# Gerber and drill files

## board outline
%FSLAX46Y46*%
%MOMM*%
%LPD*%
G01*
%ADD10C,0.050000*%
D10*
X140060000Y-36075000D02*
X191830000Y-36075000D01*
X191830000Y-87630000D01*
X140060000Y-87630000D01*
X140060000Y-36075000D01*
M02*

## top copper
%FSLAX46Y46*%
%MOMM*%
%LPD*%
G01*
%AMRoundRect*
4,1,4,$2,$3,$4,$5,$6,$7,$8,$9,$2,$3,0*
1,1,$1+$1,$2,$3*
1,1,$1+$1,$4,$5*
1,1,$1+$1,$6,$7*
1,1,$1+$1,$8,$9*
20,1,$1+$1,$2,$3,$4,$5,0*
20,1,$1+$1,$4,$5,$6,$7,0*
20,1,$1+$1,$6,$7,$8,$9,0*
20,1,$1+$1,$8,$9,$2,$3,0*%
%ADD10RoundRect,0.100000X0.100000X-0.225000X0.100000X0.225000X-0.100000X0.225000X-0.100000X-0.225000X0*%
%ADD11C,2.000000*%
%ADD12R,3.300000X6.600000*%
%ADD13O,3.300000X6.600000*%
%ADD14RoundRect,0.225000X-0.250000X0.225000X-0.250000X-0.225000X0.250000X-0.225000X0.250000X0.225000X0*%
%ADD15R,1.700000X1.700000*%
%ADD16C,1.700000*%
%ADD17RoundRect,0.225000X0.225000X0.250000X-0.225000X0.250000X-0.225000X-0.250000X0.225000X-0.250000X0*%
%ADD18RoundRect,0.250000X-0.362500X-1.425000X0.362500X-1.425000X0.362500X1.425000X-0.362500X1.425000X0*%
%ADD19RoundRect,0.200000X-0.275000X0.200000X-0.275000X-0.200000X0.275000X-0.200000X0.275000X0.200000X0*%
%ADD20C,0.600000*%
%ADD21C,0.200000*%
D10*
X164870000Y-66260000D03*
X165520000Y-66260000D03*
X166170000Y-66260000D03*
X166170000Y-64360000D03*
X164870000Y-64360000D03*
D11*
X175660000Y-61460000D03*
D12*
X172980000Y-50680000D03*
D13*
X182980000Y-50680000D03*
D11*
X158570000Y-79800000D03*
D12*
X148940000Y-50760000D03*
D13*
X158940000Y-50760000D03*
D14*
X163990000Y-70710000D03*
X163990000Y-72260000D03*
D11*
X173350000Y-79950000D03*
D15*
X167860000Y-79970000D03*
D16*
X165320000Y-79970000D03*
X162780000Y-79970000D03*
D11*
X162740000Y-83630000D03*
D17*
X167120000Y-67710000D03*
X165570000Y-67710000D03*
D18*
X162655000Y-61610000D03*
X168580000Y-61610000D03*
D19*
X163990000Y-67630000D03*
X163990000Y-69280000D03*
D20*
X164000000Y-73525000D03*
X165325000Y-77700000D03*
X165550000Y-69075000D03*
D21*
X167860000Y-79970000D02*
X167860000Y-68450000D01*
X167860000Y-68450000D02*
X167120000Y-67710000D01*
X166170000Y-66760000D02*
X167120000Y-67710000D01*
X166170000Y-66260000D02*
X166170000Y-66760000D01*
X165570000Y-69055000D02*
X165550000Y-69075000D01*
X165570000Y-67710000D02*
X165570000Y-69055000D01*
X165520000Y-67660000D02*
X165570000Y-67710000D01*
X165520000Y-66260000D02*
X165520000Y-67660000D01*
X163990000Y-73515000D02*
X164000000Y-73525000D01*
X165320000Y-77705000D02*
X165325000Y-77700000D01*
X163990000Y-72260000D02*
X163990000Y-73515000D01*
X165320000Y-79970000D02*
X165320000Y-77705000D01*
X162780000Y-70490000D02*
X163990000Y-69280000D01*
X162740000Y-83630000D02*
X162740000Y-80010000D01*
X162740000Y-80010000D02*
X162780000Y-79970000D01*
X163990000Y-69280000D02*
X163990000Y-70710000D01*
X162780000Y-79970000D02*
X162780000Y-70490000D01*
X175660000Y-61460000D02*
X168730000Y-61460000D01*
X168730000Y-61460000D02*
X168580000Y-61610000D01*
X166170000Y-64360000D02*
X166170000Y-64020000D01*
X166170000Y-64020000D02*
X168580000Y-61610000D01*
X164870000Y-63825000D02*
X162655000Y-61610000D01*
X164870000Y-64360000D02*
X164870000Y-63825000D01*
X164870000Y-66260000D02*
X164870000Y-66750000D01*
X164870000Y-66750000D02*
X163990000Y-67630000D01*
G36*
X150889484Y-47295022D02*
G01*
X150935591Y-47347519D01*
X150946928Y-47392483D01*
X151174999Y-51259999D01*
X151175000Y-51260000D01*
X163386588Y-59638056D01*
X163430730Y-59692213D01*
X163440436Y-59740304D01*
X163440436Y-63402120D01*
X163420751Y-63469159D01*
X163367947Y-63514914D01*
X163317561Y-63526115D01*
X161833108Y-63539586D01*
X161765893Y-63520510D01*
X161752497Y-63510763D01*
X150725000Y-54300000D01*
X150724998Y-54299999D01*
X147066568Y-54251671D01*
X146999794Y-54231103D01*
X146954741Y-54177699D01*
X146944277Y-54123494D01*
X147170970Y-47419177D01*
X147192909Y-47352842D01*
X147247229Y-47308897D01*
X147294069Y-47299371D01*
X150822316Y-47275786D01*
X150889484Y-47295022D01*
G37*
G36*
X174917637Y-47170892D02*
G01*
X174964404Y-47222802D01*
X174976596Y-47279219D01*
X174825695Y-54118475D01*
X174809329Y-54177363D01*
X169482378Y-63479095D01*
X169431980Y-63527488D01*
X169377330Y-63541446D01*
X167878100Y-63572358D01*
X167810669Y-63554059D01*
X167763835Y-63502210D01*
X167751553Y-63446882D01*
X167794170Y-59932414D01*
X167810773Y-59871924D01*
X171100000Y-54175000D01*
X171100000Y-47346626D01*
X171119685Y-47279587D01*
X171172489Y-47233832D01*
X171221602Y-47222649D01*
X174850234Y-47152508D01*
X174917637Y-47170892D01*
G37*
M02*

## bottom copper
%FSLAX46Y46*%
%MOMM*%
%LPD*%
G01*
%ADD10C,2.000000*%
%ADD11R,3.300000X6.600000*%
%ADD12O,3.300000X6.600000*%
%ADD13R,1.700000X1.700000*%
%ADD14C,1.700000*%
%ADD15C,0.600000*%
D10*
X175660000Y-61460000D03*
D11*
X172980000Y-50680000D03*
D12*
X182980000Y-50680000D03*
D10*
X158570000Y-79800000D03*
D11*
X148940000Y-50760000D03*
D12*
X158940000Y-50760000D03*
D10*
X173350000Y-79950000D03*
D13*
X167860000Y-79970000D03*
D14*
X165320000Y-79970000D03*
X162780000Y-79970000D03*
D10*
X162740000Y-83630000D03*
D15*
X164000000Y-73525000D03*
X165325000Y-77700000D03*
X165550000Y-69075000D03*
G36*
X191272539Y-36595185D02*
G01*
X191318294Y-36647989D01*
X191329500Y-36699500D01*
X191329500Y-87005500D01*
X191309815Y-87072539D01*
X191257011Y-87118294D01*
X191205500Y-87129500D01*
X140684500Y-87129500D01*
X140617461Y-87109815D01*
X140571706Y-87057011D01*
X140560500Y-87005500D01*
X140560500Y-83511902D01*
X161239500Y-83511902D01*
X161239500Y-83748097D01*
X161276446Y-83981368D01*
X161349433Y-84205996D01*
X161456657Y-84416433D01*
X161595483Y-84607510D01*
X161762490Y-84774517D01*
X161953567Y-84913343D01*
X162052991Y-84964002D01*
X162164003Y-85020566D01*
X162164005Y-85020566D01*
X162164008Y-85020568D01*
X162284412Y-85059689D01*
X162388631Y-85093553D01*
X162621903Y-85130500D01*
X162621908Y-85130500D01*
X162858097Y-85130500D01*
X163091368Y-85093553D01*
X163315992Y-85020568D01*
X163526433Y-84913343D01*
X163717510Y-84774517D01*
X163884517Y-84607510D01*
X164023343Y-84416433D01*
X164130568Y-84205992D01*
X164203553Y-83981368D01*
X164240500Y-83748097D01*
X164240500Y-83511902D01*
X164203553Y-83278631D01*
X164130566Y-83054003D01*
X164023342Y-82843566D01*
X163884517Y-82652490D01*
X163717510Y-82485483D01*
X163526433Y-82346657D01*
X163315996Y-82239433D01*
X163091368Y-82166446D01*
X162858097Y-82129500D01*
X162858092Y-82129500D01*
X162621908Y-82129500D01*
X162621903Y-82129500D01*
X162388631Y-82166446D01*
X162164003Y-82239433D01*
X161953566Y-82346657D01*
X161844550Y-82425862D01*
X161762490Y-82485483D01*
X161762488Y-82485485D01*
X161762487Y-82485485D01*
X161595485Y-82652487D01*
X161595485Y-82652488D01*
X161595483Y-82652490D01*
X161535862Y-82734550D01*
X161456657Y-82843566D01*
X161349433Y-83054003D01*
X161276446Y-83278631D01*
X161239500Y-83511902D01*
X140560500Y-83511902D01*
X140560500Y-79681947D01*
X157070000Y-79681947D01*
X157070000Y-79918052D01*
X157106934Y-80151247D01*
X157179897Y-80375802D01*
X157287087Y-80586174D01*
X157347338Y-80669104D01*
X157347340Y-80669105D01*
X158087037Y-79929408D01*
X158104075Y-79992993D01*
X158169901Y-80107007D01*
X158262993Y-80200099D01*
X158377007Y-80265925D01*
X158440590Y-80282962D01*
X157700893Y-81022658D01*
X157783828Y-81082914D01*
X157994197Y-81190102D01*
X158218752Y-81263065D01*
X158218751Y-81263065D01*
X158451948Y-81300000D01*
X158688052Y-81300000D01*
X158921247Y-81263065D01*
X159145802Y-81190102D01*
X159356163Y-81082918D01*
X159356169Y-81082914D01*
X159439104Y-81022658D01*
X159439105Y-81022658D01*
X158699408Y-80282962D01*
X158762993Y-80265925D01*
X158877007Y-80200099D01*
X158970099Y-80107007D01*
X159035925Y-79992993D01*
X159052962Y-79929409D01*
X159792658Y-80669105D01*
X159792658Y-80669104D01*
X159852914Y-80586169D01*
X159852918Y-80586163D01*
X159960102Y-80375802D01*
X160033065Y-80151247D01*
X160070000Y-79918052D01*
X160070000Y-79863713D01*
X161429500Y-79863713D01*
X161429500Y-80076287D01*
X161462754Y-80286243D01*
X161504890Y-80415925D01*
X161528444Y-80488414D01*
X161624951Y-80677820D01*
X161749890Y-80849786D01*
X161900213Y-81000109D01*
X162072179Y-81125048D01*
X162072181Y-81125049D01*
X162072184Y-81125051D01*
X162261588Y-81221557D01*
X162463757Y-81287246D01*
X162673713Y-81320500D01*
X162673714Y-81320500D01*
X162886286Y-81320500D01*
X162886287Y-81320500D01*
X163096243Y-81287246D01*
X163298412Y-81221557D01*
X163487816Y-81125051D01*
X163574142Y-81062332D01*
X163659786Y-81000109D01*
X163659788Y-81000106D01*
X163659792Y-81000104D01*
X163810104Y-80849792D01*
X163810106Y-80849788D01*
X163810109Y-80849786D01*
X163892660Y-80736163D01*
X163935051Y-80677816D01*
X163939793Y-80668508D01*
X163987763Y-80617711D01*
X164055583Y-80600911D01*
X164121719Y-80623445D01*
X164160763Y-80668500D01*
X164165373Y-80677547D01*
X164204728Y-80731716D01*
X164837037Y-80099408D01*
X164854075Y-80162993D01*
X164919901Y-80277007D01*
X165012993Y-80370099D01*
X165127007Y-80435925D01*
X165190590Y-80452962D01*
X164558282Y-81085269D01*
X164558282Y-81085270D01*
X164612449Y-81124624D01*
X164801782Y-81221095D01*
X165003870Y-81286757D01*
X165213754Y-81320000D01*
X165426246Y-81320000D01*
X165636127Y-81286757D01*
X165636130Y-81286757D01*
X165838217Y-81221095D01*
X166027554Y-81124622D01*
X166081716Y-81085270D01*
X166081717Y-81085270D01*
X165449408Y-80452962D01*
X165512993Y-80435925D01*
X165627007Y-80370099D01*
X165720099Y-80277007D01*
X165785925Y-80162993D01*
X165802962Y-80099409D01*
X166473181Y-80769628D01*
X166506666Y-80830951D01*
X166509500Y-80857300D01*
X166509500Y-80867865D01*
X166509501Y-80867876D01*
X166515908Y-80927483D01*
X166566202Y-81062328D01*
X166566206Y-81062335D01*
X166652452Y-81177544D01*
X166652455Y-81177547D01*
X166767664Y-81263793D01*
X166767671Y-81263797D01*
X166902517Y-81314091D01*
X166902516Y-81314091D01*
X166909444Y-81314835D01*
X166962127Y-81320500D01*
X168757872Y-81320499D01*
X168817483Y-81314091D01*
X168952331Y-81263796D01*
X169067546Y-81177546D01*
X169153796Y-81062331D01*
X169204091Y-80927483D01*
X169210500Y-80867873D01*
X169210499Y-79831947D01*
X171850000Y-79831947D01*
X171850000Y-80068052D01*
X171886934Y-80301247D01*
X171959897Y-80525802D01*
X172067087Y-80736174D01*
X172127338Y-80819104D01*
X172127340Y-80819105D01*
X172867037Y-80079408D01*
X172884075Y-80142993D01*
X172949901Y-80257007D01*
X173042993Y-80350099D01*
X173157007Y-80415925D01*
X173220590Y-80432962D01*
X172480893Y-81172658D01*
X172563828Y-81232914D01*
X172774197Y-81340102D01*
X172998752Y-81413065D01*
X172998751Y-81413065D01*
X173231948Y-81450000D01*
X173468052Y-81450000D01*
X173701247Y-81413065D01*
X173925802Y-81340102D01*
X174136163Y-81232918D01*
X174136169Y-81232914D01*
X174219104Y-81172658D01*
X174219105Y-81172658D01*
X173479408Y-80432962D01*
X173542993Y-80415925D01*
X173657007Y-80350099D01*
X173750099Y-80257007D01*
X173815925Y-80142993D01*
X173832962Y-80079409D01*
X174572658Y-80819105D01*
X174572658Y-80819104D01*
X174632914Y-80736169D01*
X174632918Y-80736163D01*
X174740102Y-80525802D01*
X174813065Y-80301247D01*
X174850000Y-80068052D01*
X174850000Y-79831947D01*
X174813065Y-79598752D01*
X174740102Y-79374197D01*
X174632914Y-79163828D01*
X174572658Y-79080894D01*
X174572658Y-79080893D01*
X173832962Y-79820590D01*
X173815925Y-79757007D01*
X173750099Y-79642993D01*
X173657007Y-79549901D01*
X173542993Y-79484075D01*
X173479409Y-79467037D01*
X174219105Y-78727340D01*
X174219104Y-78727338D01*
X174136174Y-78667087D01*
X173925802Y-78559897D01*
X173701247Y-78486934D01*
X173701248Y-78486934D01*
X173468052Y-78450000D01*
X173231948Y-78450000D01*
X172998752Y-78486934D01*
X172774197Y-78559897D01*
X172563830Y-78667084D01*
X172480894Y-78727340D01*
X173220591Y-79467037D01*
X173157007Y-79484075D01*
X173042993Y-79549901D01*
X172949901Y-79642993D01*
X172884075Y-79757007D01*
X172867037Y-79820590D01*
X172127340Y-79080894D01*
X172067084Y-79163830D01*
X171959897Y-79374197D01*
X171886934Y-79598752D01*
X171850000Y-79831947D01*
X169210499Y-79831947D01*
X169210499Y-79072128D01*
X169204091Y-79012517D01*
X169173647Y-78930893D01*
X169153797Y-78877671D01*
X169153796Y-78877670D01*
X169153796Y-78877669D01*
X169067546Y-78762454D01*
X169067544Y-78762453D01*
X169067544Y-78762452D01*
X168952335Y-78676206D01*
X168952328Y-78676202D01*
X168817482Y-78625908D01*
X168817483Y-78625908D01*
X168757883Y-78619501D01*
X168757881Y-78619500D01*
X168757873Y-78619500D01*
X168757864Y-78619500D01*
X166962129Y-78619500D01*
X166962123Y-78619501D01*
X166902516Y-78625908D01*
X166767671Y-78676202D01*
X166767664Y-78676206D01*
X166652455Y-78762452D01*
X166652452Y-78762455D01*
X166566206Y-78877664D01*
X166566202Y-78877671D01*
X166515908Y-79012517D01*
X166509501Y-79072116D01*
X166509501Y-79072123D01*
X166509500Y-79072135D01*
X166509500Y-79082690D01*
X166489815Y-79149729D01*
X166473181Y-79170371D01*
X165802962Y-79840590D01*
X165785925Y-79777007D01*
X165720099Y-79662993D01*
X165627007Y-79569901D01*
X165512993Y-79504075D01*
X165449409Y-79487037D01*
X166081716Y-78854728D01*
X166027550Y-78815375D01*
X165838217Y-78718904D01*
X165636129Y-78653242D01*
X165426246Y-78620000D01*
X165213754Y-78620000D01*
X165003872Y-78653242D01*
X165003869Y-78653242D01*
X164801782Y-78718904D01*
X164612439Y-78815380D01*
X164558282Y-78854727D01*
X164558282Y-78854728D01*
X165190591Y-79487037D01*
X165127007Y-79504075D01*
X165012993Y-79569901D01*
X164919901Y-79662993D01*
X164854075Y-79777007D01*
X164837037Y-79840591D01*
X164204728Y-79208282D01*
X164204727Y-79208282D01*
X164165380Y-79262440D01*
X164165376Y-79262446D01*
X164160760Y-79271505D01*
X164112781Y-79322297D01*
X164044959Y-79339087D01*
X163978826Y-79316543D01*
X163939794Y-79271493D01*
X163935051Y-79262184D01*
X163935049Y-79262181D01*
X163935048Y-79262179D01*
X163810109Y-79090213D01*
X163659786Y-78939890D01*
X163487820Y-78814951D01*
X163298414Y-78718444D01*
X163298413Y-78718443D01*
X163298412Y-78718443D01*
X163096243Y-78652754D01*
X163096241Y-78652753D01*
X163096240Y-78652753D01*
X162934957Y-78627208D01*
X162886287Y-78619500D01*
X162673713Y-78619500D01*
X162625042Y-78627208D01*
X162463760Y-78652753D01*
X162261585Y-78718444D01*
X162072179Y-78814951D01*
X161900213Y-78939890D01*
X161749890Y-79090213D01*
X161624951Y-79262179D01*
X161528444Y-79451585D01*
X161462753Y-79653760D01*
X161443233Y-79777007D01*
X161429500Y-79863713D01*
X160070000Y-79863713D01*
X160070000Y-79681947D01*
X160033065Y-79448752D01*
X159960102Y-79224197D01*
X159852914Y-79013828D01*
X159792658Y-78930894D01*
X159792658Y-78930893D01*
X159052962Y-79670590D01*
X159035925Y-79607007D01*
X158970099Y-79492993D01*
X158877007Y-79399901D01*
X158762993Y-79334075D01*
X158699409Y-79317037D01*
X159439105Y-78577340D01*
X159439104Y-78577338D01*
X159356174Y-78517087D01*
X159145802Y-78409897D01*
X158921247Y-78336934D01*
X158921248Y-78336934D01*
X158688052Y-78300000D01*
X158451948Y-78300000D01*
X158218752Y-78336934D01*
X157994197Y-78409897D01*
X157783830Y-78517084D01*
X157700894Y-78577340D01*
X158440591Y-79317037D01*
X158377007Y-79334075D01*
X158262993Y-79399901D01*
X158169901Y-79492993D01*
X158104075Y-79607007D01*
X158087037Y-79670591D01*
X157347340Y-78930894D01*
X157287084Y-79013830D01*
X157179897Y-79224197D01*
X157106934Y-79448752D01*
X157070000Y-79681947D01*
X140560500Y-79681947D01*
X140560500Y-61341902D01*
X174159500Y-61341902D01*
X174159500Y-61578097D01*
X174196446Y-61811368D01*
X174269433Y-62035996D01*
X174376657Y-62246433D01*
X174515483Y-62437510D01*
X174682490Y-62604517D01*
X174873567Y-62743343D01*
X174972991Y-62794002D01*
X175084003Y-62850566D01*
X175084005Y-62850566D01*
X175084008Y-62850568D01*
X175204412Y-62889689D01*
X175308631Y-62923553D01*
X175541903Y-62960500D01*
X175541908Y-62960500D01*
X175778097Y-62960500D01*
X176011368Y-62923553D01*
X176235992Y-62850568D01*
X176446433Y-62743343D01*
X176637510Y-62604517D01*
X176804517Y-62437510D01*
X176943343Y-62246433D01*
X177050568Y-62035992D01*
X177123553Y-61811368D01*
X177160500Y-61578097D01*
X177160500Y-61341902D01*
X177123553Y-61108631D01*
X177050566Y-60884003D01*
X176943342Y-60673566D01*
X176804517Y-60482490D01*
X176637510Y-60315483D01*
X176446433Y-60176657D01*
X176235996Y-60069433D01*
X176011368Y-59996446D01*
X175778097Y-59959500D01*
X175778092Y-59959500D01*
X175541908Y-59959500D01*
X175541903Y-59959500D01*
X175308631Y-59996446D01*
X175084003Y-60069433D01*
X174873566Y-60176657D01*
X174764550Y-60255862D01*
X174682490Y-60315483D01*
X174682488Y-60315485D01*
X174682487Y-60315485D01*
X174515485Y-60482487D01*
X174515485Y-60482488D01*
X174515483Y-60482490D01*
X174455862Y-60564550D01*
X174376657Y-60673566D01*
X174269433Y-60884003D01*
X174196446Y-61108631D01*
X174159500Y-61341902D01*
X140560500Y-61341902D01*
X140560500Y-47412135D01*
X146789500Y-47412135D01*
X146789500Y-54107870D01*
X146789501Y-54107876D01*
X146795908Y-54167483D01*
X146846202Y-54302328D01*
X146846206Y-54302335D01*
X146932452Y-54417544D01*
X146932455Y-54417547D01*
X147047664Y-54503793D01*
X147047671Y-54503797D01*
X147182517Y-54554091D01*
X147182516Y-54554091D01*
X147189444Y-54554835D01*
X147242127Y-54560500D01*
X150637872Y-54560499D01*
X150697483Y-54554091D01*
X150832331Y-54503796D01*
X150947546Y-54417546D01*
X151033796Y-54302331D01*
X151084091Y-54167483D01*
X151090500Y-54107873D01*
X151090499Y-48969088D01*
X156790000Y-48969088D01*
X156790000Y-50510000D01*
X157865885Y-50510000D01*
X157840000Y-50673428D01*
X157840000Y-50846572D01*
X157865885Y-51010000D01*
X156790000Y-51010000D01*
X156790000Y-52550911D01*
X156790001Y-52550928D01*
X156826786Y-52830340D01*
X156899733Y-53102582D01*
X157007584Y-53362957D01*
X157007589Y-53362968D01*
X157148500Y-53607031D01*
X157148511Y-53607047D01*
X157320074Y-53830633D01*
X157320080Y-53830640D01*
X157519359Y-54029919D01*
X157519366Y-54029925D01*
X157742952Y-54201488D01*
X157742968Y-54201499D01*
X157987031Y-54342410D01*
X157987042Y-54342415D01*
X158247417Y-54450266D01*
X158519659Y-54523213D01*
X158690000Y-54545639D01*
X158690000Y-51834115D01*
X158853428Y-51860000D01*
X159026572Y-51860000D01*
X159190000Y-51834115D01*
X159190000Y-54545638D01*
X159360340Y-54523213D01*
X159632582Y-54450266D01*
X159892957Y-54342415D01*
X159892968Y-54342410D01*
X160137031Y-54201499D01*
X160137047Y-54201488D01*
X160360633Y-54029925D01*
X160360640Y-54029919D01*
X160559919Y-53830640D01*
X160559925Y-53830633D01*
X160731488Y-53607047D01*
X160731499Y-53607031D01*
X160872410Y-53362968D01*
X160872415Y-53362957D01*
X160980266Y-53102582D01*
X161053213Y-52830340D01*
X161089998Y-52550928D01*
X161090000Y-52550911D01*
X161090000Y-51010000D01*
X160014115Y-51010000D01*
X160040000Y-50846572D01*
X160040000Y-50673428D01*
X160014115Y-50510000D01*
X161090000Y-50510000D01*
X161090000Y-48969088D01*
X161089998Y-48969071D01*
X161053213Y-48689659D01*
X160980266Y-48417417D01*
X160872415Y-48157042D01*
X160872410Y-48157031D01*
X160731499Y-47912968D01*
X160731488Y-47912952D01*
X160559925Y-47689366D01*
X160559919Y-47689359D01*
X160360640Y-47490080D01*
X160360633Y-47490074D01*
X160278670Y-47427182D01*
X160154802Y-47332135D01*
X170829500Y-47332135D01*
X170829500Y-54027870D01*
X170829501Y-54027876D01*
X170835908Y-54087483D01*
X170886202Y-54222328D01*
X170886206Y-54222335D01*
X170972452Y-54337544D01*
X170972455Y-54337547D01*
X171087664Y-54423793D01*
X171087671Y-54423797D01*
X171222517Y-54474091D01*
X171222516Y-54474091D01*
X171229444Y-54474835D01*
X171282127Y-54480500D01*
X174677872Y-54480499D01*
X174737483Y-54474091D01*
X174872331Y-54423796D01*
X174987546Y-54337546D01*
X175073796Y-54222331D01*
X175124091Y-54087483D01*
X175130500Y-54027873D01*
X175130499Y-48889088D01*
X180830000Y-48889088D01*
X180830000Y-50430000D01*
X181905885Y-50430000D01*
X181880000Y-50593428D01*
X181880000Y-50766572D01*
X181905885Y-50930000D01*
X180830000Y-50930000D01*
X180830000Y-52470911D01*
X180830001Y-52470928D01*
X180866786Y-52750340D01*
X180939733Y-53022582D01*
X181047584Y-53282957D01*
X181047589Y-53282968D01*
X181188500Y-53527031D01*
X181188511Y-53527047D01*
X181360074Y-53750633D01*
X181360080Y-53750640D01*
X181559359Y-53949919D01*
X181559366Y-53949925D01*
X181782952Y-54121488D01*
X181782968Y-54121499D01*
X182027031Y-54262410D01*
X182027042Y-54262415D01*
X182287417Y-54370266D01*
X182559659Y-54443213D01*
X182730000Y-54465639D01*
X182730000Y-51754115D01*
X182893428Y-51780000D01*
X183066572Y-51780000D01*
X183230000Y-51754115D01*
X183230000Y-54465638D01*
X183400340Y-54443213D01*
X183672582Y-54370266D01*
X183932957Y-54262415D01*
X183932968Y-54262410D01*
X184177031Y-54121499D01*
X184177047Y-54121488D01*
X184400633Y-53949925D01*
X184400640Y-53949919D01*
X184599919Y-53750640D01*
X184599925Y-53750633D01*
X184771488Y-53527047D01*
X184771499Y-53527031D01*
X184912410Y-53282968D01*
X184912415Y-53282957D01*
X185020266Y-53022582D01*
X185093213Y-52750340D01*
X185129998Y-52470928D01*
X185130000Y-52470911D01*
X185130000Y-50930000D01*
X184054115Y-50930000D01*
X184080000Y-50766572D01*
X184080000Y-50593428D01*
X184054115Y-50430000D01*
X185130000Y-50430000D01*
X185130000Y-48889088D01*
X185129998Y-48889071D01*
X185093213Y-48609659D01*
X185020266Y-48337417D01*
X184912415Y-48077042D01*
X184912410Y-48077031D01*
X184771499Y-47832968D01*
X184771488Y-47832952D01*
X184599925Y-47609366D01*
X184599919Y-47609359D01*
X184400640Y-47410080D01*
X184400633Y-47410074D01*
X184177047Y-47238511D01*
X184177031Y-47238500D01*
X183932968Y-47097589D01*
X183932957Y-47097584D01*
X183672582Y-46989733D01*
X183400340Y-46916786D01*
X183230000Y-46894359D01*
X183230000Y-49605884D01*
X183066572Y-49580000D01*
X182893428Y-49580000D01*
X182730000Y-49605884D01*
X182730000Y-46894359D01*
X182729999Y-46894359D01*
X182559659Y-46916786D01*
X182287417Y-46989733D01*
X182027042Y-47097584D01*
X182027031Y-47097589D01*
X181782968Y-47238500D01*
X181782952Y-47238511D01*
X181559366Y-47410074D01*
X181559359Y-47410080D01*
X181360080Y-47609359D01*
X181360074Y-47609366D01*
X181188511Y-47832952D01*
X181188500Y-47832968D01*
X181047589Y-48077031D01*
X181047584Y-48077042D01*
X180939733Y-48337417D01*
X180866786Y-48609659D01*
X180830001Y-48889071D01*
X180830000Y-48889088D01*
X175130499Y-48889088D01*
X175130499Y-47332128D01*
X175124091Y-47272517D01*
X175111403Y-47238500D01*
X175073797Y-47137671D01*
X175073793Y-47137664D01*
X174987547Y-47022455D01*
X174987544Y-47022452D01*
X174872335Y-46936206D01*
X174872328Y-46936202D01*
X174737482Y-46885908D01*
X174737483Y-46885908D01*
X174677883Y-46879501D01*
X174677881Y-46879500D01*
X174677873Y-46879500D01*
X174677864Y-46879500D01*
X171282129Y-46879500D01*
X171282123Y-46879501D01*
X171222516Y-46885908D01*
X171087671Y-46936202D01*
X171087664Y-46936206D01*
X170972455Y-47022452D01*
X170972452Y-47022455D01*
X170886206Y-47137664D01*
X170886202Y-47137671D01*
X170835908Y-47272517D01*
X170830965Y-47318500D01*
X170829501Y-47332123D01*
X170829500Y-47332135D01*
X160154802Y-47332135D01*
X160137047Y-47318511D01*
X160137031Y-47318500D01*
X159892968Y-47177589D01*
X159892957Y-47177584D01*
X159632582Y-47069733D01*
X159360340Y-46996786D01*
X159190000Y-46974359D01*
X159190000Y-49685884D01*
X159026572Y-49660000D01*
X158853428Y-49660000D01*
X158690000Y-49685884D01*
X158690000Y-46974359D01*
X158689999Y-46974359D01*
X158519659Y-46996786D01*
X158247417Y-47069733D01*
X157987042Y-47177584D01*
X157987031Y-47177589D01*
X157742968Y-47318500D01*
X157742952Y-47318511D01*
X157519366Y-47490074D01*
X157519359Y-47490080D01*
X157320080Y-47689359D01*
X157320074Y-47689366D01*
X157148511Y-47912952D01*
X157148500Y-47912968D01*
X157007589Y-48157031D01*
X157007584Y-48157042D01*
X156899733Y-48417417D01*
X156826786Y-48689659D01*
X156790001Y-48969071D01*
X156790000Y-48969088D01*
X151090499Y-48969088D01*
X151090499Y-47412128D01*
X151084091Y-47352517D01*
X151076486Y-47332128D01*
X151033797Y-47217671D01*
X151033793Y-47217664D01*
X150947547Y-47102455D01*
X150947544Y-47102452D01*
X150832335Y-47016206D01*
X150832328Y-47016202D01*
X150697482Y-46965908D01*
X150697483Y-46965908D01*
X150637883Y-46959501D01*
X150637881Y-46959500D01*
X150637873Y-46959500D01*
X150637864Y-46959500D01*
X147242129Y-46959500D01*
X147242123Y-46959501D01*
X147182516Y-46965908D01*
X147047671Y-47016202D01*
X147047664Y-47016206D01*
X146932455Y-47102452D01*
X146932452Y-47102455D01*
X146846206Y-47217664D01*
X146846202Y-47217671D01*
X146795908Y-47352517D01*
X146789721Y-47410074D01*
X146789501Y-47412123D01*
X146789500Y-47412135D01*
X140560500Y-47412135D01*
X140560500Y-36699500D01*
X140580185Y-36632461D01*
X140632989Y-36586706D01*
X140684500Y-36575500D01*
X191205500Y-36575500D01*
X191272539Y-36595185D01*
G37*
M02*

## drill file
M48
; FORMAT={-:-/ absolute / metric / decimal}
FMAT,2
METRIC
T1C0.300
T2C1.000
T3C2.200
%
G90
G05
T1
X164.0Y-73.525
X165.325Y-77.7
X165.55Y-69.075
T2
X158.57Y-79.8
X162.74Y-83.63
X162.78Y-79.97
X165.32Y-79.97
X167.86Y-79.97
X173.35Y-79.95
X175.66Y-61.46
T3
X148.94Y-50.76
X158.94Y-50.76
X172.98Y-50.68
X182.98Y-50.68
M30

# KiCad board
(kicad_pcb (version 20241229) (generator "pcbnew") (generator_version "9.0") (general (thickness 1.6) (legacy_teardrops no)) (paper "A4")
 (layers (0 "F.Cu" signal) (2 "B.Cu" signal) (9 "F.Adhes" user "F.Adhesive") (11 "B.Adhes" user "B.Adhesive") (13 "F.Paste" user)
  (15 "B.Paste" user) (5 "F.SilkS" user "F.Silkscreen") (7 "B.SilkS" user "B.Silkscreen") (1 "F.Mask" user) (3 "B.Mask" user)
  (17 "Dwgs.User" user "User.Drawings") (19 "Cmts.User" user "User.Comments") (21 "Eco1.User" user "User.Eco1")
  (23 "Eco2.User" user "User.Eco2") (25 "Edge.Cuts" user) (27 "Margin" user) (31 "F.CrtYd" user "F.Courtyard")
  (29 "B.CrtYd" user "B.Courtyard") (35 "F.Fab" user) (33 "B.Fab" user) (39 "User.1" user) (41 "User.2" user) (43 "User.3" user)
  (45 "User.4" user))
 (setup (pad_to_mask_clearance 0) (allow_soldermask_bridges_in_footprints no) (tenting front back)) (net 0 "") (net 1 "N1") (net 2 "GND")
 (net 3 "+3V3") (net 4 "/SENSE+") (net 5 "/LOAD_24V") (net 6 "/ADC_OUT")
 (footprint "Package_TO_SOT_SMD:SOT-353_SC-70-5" (layer "F.Cu") (at 165.52 65.31 90)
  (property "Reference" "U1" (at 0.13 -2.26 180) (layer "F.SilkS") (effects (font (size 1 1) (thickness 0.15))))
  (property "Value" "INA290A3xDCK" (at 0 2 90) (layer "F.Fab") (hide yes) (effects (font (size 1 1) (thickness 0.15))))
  (pad "1" smd roundrect (at -0.95 -0.65 90) (size 0.65 0.4) (layers "F.Cu" "F.Mask" "F.Paste") (roundrect_rratio 0.25) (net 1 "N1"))
  (pad "2" smd roundrect (at -0.95 0 90) (size 0.65 0.4) (layers "F.Cu" "F.Mask" "F.Paste") (roundrect_rratio 0.25) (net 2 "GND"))
  (pad "3" smd roundrect (at -0.95 0.65 90) (size 0.65 0.4) (layers "F.Cu" "F.Mask" "F.Paste") (roundrect_rratio 0.25) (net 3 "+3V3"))
  (pad "4" smd roundrect (at 0.95 0.65 90) (size 0.65 0.4) (layers "F.Cu" "F.Mask" "F.Paste") (roundrect_rratio 0.25) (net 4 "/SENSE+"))
  (pad "5" smd roundrect (at 0.95 -0.65 90) (size 0.65 0.4) (layers "F.Cu" "F.Mask" "F.Paste") (roundrect_rratio 0.25) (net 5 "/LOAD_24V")))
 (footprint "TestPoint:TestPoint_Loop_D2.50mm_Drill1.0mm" (layer "F.Cu") (at 175.66 61.46)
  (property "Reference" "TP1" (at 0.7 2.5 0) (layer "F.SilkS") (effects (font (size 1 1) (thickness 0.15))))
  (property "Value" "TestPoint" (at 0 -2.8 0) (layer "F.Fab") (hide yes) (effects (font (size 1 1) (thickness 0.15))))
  (pad "1" thru_hole circle (at 0 0) (size 2 2) (drill 1) (layers "*.Cu" "*.Mask") (remove_unused_layers no) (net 4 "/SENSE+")))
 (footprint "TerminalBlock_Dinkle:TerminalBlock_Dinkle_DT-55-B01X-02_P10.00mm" (layer "F.Cu") (at 172.98 50.68)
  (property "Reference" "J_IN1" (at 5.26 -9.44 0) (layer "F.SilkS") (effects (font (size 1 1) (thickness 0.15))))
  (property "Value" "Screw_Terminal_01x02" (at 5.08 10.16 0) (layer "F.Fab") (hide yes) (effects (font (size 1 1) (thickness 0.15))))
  (pad "1" thru_hole rect (at 0 0) (size 3.3 6.6) (drill 2.2) (layers "*.Cu" "*.Mask") (remove_unused_layers no) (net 4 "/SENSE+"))
  (pad "2" thru_hole oval (at 10 0) (size 3.3 6.6) (drill 2.2) (layers "*.Cu" "*.Mask") (remove_unused_layers no) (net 2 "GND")))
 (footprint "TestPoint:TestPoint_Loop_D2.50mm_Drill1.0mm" (layer "F.Cu") (at 158.57 79.8)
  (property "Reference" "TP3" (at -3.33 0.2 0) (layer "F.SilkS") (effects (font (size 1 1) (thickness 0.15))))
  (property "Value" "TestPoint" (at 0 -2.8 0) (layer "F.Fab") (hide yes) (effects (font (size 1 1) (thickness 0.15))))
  (pad "1" thru_hole circle (at 0 0) (size 2 2) (drill 1) (layers "*.Cu" "*.Mask") (remove_unused_layers no) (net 2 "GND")))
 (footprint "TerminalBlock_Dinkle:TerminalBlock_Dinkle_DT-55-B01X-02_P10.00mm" (layer "F.Cu") (at 148.94 50.76)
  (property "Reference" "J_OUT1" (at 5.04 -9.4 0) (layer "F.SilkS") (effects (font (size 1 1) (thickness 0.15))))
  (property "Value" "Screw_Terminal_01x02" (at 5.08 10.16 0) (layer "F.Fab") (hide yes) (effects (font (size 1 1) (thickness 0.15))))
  (pad "1" thru_hole rect (at 0 0) (size 3.3 6.6) (drill 2.2) (layers "*.Cu" "*.Mask") (remove_unused_layers no) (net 5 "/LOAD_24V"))
  (pad "2" thru_hole oval (at 10 0) (size 3.3 6.6) (drill 2.2) (layers "*.Cu" "*.Mask") (remove_unused_layers no) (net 2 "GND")))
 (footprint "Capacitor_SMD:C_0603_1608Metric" (layer "F.Cu") (at 163.99 71.485 -90)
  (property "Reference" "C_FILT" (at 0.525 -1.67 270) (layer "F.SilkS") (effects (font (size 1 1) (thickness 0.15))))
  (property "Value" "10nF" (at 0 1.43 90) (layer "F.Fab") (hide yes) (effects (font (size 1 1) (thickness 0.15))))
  (pad "1" smd roundrect (at -0.775 0 270) (size 0.9 0.95) (layers "F.Cu" "F.Mask" "F.Paste") (roundrect_rratio 0.25) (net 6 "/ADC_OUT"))
  (pad "2" smd roundrect (at 0.775 0 270) (size 0.9 0.95) (layers "F.Cu" "F.Mask" "F.Paste") (roundrect_rratio 0.25) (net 2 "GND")))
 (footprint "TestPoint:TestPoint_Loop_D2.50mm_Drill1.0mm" (layer "F.Cu") (at 173.35 79.95)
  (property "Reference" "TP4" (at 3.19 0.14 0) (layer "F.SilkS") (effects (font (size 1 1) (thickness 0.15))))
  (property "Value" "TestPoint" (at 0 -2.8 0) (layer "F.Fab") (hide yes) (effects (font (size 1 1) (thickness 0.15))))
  (pad "1" thru_hole circle (at 0 0) (size 2 2) (drill 1) (layers "*.Cu" "*.Mask") (remove_unused_layers no) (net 2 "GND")))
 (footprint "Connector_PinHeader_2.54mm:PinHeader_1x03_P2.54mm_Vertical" (layer "F.Cu") (at 167.86 79.97 -90)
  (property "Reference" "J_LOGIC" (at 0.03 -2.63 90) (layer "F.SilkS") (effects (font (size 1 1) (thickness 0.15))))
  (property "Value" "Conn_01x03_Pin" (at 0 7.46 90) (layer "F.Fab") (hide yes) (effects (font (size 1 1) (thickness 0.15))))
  (pad "1" thru_hole rect (at 0 0 270) (size 1.7 1.7) (drill 1) (layers "*.Cu" "*.Mask") (remove_unused_layers no) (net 3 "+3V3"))
  (pad "2" thru_hole circle (at 0 2.54 270) (size 1.7 1.7) (drill 1) (layers "*.Cu" "*.Mask") (remove_unused_layers no) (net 2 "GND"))
  (pad "3" thru_hole circle (at 0 5.08 270) (size 1.7 1.7) (drill 1) (layers "*.Cu" "*.Mask") (remove_unused_layers no) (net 6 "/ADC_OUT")))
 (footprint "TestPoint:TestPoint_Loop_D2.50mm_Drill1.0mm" (layer "F.Cu") (at 162.74 83.63)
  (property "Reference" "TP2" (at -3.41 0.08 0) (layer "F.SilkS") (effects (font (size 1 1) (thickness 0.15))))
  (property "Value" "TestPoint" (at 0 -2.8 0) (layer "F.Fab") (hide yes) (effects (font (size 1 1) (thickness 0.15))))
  (pad "1" thru_hole circle (at 0 0) (size 2 2) (drill 1) (layers "*.Cu" "*.Mask") (remove_unused_layers no) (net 6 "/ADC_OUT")))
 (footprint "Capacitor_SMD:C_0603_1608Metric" (layer "F.Cu") (at 166.345 67.71 180)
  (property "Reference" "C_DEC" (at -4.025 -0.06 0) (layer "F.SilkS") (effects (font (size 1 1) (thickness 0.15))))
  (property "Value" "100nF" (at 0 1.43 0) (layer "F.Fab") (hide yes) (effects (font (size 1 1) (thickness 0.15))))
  (pad "1" smd roundrect (at -0.775 0 180) (size 0.9 0.95) (layers "F.Cu" "F.Mask" "F.Paste") (roundrect_rratio 0.25) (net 3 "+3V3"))
  (pad "2" smd roundrect (at 0.775 0 180) (size 0.9 0.95) (layers "F.Cu" "F.Mask" "F.Paste") (roundrect_rratio 0.25) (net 2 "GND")))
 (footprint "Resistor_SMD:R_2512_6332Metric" (layer "F.Cu") (at 165.6175 61.61)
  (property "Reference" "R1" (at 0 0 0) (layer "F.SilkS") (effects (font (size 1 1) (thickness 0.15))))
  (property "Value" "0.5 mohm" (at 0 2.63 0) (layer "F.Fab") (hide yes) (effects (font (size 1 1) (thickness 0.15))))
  (pad "1" smd roundrect (at -2.9625 0) (size 1.225 3.35) (layers "F.Cu" "F.Mask" "F.Paste") (roundrect_rratio 0.204082) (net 5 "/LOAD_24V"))
  (pad "2" smd roundrect (at 2.9625 0) (size 1.225 3.35) (layers "F.Cu" "F.Mask" "F.Paste") (roundrect_rratio 0.204082) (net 4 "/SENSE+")))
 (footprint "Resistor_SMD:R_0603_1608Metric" (layer "F.Cu") (at 163.99 68.455 -90)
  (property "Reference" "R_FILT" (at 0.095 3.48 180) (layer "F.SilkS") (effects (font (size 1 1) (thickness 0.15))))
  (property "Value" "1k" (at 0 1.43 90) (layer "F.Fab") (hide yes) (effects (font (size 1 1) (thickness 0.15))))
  (pad "1" smd roundrect (at -0.825 0 270) (size 0.8 0.95) (layers "F.Cu" "F.Mask" "F.Paste") (roundrect_rratio 0.25) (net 1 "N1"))
  (pad "2" smd roundrect (at 0.825 0 270) (size 0.8 0.95) (layers "F.Cu" "F.Mask" "F.Paste") (roundrect_rratio 0.25) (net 6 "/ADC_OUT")))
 (gr_rect (start 140.06 36.075) (end 191.83 87.63) (stroke (width 0.05) (type default)) (fill no) (layer "Edge.Cuts"))
 (segment (start 167.86 79.97) (end 167.86 68.45) (width 0.2) (layer "F.Cu") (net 3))
 (segment (start 167.86 68.45) (end 167.12 67.71) (width 0.2) (layer "F.Cu") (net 3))
 (segment (start 166.17 66.76) (end 167.12 67.71) (width 0.2) (layer "F.Cu") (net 3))
 (segment (start 166.17 66.26) (end 166.17 66.76) (width 0.2) (layer "F.Cu") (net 3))
 (segment (start 165.57 69.055) (end 165.55 69.075) (width 0.2) (layer "F.Cu") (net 2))
 (segment (start 165.57 67.71) (end 165.57 69.055) (width 0.2) (layer "F.Cu") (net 2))
 (segment (start 165.52 67.66) (end 165.57 67.71) (width 0.2) (layer "F.Cu") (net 2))
 (segment (start 165.52 66.26) (end 165.52 67.66) (width 0.2) (layer "F.Cu") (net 2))
 (segment (start 163.99 73.515) (end 164 73.525) (width 0.2) (layer "F.Cu") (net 2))
 (segment (start 165.32 77.705) (end 165.325 77.7) (width 0.2) (layer "F.Cu") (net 2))
 (segment (start 163.99 72.26) (end 163.99 73.515) (width 0.2) (layer "F.Cu") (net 2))
 (segment (start 165.32 79.97) (end 165.32 77.705) (width 0.2) (layer "F.Cu") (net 2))
 (via (at 164 73.525) (size 0.6) (drill 0.3) (layers "F.Cu" "B.Cu") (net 2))
 (via (at 165.325 77.7) (size 0.6) (drill 0.3) (layers "F.Cu" "B.Cu") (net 2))
 (via (at 165.55 69.075) (size 0.6) (drill 0.3) (layers "F.Cu" "B.Cu") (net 2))
 (segment (start 162.78 70.49) (end 163.99 69.28) (width 0.2) (layer "F.Cu") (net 6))
 (segment (start 162.74 83.63) (end 162.74 80.01) (width 0.2) (layer "F.Cu") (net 6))
 (segment (start 162.74 80.01) (end 162.78 79.97) (width 0.2) (layer "F.Cu") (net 6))
 (segment (start 163.99 69.28) (end 163.99 70.71) (width 0.2) (layer "F.Cu") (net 6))
 (segment (start 162.78 79.97) (end 162.78 70.49) (width 0.2) (layer "F.Cu") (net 6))
 (segment (start 175.66 61.46) (end 168.73 61.46) (width 0.2) (layer "F.Cu") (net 4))
 (segment (start 168.73 61.46) (end 168.58 61.61) (width 0.2) (layer "F.Cu") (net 4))
 (segment (start 166.17 64.36) (end 166.17 64.02) (width 0.2) (layer "F.Cu") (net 4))
 (segment (start 166.17 64.02) (end 168.58 61.61) (width 0.2) (layer "F.Cu") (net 4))
 (segment (start 164.87 63.825) (end 162.655 61.61) (width 0.2) (layer "F.Cu") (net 5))
 (segment (start 164.87 64.36) (end 164.87 63.825) (width 0.2) (layer "F.Cu") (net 5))
 (segment (start 164.87 66.26) (end 164.87 66.75) (width 0.2) (layer "F.Cu") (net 1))
 (segment (start 164.87 66.75) (end 163.99 67.63) (width 0.2) (layer "F.Cu") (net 1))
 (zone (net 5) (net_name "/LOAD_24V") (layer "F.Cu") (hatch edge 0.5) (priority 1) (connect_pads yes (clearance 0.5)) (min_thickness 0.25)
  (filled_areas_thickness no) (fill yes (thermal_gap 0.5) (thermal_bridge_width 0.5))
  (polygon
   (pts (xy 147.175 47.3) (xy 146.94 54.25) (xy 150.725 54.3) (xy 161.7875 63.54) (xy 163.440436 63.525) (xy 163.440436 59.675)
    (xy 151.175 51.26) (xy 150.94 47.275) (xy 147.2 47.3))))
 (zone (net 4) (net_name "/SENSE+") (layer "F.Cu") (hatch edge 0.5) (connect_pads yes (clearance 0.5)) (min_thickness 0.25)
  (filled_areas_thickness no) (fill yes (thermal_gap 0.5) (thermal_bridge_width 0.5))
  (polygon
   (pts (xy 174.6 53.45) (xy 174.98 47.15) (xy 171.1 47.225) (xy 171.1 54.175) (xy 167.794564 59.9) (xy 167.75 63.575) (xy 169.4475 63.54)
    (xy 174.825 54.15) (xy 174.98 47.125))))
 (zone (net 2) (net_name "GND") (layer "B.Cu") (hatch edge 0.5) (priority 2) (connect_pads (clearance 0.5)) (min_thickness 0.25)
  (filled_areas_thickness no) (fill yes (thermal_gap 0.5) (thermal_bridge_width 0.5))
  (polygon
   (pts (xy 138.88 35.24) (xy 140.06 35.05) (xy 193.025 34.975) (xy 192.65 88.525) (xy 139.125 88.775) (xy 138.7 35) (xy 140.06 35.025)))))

